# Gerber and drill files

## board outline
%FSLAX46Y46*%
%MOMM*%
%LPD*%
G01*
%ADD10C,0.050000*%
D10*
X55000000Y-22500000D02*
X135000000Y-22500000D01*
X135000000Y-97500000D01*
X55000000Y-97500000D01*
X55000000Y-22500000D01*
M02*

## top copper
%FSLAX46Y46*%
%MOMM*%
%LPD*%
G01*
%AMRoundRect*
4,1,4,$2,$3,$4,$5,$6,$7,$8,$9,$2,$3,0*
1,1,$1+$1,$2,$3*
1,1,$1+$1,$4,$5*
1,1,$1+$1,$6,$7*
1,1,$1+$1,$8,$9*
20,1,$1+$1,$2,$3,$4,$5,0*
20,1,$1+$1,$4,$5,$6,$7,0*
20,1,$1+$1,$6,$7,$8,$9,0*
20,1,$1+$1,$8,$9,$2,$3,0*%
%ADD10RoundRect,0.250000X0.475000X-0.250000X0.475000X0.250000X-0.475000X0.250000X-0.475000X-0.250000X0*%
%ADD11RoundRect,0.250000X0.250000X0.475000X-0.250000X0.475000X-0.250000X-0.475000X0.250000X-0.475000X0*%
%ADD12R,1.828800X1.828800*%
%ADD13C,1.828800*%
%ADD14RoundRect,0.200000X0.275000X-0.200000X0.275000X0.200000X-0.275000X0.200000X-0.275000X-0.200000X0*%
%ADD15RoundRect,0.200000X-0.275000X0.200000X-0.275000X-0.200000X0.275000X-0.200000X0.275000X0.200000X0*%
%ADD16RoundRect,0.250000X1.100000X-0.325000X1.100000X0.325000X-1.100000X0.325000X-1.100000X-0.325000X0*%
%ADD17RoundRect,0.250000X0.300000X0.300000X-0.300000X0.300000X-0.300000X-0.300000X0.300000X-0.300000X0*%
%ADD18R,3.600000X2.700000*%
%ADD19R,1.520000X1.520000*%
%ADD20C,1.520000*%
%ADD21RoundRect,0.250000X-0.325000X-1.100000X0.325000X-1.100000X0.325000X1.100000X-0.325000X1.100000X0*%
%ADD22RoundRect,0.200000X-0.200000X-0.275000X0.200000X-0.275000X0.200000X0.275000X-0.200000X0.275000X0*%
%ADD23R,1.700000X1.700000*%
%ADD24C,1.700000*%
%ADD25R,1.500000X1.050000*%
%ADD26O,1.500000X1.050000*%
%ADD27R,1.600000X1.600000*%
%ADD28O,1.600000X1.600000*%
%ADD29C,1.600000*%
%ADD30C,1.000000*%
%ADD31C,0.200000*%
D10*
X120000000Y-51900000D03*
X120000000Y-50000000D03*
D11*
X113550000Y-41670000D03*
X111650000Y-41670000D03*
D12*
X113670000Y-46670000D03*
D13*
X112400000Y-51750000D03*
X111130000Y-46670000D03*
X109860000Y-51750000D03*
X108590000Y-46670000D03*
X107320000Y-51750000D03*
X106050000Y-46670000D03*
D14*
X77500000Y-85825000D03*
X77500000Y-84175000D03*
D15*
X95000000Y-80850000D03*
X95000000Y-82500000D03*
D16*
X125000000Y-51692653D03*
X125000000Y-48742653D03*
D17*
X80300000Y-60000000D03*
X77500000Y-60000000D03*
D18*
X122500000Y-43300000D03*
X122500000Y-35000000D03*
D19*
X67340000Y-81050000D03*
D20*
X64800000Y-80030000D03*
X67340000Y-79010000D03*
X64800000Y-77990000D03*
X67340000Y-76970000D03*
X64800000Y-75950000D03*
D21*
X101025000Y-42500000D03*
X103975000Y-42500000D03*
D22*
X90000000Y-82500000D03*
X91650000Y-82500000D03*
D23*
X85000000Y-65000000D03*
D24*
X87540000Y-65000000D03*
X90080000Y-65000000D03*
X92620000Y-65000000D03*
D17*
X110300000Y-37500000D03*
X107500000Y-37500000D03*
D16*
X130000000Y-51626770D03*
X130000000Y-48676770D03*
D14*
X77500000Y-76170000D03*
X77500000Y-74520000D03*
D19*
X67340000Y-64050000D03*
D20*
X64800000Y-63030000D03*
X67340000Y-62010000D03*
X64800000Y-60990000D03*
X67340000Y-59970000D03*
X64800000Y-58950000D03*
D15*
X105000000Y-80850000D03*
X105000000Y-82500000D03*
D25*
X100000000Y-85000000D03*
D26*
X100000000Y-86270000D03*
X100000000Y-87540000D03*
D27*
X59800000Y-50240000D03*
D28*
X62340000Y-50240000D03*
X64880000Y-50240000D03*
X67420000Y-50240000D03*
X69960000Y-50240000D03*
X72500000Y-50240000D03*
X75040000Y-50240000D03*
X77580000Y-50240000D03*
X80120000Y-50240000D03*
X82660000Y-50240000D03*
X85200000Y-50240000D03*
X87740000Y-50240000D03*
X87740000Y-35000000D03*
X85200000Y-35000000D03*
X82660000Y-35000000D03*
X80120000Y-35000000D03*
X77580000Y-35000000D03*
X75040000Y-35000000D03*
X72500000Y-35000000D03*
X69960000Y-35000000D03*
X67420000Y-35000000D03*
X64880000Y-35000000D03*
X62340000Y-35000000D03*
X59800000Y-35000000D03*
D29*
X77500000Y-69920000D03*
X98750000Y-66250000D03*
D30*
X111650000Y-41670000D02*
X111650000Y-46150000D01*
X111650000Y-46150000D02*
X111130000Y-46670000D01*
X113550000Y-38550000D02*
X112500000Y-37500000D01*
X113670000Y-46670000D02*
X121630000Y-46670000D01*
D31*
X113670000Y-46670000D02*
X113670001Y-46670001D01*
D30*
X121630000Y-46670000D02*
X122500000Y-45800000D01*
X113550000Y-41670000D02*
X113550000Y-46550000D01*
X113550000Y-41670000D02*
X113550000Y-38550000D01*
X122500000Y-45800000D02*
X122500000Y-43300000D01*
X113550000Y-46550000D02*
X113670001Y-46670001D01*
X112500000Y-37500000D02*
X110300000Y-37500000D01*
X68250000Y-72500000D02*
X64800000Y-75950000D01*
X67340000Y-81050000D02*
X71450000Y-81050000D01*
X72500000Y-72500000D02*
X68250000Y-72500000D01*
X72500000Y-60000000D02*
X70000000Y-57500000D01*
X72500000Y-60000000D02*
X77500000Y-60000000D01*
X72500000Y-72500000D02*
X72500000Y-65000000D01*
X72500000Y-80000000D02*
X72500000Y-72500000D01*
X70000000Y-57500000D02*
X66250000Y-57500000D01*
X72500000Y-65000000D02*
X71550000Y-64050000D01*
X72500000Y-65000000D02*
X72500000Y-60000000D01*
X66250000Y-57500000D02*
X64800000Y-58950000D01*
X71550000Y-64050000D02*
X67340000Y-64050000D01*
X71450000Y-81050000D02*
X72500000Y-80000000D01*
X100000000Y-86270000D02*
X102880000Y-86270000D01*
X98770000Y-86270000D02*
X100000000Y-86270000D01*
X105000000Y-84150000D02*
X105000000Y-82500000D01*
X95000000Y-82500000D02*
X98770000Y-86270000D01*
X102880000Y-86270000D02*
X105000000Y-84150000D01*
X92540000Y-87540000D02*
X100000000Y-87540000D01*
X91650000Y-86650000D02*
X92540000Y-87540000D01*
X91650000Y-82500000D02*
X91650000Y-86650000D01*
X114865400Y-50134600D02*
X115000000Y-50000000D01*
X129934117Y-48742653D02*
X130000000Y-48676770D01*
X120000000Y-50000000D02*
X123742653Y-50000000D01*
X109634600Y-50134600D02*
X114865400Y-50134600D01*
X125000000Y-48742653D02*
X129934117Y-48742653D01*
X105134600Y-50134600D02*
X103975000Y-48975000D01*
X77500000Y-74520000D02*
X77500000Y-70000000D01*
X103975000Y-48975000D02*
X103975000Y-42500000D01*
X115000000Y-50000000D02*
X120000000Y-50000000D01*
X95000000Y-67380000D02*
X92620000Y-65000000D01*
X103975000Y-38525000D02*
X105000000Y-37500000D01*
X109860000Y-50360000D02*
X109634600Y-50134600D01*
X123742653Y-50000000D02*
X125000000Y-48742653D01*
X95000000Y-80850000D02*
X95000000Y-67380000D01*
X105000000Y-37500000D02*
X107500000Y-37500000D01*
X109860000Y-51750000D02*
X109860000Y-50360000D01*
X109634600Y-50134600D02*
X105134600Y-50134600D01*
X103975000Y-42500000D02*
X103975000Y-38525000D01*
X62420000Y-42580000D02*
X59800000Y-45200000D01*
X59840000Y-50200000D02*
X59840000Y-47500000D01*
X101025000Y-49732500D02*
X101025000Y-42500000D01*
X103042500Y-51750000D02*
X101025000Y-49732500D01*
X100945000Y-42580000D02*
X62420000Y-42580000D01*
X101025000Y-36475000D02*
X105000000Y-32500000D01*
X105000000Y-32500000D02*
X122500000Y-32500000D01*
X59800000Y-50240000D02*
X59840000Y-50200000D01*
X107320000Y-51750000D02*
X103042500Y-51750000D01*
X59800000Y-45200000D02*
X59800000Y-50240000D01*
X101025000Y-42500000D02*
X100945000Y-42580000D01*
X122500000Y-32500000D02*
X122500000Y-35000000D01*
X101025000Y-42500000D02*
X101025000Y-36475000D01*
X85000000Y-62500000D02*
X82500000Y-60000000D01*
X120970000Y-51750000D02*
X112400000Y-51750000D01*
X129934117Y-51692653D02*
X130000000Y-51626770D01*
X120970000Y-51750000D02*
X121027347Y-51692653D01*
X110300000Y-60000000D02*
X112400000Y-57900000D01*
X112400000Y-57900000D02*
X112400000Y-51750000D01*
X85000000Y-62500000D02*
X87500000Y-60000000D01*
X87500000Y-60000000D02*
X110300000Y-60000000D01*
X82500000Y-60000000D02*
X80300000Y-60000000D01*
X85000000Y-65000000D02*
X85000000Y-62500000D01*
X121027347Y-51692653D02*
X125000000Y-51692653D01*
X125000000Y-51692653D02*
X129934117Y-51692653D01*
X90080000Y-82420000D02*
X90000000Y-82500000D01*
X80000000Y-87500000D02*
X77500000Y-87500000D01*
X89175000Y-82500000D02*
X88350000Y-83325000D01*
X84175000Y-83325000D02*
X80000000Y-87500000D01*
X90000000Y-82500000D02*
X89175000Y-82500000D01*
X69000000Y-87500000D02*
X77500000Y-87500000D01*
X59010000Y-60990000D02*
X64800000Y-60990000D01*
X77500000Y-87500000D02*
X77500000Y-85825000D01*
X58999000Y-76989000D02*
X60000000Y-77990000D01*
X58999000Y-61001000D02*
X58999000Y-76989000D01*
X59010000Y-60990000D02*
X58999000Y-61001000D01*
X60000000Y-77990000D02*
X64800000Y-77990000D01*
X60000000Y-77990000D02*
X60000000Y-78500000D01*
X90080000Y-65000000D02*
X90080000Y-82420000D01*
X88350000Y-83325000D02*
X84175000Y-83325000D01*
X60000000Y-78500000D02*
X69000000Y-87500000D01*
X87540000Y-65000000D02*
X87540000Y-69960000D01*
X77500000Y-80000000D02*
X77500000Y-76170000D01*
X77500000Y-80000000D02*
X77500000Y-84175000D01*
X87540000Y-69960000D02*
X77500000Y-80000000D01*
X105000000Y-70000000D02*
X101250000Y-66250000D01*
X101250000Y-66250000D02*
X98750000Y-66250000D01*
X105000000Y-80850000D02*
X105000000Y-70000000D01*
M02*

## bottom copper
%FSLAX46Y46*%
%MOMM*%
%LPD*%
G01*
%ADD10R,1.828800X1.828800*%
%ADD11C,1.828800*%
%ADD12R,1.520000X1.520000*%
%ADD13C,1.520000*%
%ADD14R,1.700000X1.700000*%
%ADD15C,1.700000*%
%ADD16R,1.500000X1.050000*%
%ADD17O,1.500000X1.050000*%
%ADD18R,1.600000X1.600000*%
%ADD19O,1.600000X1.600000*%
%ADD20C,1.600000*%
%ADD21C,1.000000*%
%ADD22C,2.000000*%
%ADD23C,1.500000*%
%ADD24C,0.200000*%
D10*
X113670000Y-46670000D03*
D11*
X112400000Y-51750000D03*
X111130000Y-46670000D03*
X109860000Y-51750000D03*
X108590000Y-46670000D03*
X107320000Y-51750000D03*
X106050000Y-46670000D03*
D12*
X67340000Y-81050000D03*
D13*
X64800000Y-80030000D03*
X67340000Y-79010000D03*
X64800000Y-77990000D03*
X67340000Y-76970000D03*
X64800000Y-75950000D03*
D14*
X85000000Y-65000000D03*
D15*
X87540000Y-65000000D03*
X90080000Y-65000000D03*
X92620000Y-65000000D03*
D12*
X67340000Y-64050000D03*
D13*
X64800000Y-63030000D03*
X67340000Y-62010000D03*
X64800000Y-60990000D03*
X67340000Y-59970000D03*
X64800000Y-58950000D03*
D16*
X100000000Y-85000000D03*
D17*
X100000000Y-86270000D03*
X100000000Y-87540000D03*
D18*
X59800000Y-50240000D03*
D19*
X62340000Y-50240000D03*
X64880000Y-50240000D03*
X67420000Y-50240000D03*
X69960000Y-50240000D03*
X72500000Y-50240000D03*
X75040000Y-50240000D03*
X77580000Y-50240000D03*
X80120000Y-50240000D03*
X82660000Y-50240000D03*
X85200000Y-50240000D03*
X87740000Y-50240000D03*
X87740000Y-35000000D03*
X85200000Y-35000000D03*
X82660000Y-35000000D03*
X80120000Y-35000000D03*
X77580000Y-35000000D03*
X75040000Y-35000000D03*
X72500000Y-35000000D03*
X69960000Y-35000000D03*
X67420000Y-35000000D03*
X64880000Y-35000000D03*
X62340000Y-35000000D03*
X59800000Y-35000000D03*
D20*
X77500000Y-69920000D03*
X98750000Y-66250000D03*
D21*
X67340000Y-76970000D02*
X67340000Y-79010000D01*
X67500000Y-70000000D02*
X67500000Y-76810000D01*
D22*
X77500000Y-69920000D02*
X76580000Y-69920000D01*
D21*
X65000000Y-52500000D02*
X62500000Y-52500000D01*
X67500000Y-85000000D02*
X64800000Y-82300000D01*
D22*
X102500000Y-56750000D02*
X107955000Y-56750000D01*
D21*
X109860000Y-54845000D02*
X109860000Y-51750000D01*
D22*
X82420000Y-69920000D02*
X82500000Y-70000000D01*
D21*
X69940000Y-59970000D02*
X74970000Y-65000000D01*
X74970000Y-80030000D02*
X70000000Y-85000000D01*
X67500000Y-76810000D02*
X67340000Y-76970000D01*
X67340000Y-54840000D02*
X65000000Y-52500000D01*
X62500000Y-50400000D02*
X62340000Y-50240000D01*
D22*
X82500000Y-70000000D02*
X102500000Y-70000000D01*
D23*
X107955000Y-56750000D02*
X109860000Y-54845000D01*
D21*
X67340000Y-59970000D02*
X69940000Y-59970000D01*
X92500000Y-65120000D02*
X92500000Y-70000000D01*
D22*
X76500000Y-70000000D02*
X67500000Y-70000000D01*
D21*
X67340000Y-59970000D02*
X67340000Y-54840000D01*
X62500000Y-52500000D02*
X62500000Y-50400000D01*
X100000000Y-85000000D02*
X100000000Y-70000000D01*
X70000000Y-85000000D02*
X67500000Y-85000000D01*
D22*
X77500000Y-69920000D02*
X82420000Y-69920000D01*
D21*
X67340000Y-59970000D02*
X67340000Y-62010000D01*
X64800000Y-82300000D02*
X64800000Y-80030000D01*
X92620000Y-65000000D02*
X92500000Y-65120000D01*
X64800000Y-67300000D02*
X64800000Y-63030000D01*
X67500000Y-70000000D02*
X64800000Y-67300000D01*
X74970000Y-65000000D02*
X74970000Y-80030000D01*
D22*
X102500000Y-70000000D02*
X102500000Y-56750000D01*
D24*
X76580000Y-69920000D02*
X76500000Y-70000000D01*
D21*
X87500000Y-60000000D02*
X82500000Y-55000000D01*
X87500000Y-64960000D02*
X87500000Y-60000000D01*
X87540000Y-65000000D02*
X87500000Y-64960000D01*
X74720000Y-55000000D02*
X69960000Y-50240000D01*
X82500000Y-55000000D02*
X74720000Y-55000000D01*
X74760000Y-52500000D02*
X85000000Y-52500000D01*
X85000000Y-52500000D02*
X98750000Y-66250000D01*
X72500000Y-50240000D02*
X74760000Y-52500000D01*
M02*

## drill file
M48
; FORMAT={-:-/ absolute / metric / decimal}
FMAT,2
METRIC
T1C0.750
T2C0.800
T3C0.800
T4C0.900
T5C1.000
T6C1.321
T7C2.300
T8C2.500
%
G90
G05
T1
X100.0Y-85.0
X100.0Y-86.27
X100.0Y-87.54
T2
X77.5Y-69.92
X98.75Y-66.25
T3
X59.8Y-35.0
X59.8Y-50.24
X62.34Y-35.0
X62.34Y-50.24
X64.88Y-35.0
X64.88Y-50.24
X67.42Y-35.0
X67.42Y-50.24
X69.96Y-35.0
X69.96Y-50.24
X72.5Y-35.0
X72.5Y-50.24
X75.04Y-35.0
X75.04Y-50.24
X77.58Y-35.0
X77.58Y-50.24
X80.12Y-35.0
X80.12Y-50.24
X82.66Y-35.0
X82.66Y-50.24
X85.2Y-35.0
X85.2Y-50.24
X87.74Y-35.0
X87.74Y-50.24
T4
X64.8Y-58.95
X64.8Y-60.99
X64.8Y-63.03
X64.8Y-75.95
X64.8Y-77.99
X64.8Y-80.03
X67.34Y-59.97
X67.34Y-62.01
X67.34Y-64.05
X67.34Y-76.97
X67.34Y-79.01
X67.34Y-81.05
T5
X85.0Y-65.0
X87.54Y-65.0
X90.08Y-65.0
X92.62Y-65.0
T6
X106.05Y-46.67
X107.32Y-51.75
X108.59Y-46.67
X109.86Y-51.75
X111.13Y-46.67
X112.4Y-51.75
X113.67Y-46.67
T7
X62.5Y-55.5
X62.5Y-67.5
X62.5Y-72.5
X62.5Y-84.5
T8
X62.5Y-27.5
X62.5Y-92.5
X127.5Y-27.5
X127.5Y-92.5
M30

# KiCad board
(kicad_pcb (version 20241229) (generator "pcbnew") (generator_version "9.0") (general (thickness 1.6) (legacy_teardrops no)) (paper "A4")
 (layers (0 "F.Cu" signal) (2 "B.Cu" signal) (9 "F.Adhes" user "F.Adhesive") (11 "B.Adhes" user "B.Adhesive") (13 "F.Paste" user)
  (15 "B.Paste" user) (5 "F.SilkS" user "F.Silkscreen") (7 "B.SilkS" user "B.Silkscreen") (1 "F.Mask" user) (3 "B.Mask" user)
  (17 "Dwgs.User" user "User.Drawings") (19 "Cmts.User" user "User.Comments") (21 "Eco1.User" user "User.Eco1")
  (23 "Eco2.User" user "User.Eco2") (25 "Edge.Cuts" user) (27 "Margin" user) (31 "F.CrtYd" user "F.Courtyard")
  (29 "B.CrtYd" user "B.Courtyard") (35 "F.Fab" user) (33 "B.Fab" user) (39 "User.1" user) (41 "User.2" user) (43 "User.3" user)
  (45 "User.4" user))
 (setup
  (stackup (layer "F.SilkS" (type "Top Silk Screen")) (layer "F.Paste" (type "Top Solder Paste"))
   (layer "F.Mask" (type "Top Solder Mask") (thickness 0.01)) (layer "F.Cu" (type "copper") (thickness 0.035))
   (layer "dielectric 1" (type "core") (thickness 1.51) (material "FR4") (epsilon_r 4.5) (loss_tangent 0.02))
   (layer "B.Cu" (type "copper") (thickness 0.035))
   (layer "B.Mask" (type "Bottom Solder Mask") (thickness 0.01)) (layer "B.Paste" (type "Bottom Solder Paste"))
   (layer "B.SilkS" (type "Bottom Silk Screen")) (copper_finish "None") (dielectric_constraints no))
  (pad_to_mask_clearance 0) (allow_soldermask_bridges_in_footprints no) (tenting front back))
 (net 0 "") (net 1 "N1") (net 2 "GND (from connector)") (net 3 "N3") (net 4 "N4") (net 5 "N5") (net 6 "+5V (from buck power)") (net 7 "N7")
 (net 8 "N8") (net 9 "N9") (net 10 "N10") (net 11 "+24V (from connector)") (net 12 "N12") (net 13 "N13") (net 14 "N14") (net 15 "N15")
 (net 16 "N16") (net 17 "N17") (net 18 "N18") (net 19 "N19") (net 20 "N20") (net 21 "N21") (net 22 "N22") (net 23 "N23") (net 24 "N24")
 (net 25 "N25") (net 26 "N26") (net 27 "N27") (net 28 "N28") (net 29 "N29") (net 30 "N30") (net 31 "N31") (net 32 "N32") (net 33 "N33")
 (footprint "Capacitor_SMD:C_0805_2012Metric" (layer "F.Cu") (at 120 50.95 90)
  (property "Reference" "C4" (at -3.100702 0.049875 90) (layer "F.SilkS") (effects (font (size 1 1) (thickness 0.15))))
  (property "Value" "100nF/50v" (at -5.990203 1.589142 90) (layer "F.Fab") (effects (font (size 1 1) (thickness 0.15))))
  (pad "1" smd roundrect (at -0.95 0 90) (size 1 1.45) (layers "F.Cu" "F.Mask" "F.Paste") (roundrect_rratio 0.25) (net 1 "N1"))
  (pad "2" smd roundrect (at 0.95 0 90) (size 1 1.45) (layers "F.Cu" "F.Mask" "F.Paste") (roundrect_rratio 0.25)
   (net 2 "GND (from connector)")))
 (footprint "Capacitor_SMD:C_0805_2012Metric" (layer "F.Cu") (at 112.6 41.67 180)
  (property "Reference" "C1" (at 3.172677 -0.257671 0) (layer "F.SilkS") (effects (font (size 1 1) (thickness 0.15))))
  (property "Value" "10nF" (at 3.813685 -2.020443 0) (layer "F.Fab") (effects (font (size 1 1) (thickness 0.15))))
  (pad "1" smd roundrect (at -0.95 0 180) (size 1 1.45) (layers "F.Cu" "F.Mask" "F.Paste") (roundrect_rratio 0.25) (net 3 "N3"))
  (pad "2" smd roundrect (at 0.95 0 180) (size 1 1.45) (layers "F.Cu" "F.Mask" "F.Paste") (roundrect_rratio 0.25) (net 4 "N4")))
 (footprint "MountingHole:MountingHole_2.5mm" (layer "F.Cu") (at 62.5 27.5)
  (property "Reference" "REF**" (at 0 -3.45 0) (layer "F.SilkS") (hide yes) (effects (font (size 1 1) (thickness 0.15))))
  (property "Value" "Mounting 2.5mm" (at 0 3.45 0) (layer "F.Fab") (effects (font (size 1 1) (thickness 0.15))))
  (pad "" np_thru_hole circle (at 0 0) (size 2.5 2.5) (drill 2.5) (layers "*.Cu" "*.Mask")))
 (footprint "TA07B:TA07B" (layer "F.Cu") (at 106.05 57.8714 180)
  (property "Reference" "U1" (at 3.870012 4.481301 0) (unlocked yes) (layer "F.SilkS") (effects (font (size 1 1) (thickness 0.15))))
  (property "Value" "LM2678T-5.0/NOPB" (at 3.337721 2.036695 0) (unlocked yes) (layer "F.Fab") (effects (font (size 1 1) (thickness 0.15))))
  (pad "1" thru_hole rect (at -7.62 11.2014 180) (size 1.8288 1.8288) (drill 1.3208) (layers "*.Cu" "*.Mask") (remove_unused_layers no)
   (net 3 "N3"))
  (pad "2" thru_hole circle (at -6.35 6.1214 180) (size 1.8288 1.8288) (drill 1.3208) (layers "*.Cu" "*.Mask") (remove_unused_layers no)
   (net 1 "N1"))
  (pad "3" thru_hole circle (at -5.08 11.2014 180) (size 1.8288 1.8288) (drill 1.3208) (layers "*.Cu" "*.Mask") (remove_unused_layers no)
   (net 4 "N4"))
  (pad "4" thru_hole circle (at -3.81 6.1214 180) (size 1.8288 1.8288) (drill 1.3208) (layers "*.Cu" "*.Mask") (remove_unused_layers no)
   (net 2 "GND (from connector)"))
  (pad "5" thru_hole circle (at -2.54 11.2014 180) (size 1.8288 1.8288) (drill 1.3208) (layers "*.Cu" "*.Mask") (remove_unused_layers no)
   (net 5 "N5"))
  (pad "6" thru_hole circle (at -1.27 6.1214 180) (size 1.8288 1.8288) (drill 1.3208) (layers "*.Cu" "*.Mask") (remove_unused_layers no)
   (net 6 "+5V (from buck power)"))
  (pad "7" thru_hole circle (at 0 11.2014 180) (size 1.8288 1.8288) (drill 1.3208) (layers "*.Cu" "*.Mask") (remove_unused_layers no)
   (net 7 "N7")))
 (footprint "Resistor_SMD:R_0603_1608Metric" (layer "F.Cu") (at 77.5 85 90)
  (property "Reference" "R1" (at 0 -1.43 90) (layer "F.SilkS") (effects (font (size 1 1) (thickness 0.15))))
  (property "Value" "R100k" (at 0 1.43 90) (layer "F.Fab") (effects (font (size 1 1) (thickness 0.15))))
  (pad "1" smd roundrect (at -0.825 0 90) (size 0.8 0.95) (layers "F.Cu" "F.Mask" "F.Paste") (roundrect_rratio 0.25) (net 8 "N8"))
  (pad "2" smd roundrect (at 0.825 0 90) (size 0.8 0.95) (layers "F.Cu" "F.Mask" "F.Paste") (roundrect_rratio 0.25) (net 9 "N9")))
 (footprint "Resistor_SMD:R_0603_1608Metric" (layer "F.Cu") (at 95 81.675 -90)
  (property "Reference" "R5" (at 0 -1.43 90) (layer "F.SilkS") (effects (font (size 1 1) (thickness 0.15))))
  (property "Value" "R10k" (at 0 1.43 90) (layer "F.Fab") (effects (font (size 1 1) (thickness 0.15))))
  (pad "1" smd roundrect (at -0.825 0 270) (size 0.8 0.95) (layers "F.Cu" "F.Mask" "F.Paste") (roundrect_rratio 0.25)
   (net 2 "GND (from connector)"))
  (pad "2" smd roundrect (at 0.825 0 270) (size 0.8 0.95) (layers "F.Cu" "F.Mask" "F.Paste") (roundrect_rratio 0.25) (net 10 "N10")))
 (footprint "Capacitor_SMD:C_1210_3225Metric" (layer "F.Cu") (at 125 50.217653 90)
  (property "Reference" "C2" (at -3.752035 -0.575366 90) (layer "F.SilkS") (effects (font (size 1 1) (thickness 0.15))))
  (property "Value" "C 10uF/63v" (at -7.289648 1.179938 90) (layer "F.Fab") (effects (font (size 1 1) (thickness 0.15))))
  (pad "1" smd roundrect (at -1.475 0 90) (size 1.15 2.7) (layers "F.Cu" "F.Mask" "F.Paste") (roundrect_rratio 0.217391) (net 1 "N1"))
  (pad "2" smd roundrect (at 1.475 0 90) (size 1.15 2.7) (layers "F.Cu" "F.Mask" "F.Paste") (roundrect_rratio 0.217391)
   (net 2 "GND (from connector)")))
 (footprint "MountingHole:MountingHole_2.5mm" (layer "F.Cu") (at 127.5 27.5)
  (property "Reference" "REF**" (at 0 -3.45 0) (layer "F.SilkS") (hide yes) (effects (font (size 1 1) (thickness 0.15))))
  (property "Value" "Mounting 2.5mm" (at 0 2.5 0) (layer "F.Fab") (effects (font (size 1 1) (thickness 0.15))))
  (pad "" np_thru_hole circle (at 0 0) (size 2.5 2.5) (drill 2.5) (layers "*.Cu" "*.Mask")))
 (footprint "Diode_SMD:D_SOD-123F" (layer "F.Cu") (at 78.9 60 180)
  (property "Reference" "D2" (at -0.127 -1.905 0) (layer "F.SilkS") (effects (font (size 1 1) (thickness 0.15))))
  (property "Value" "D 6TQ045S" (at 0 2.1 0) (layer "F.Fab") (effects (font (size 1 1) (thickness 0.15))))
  (pad "1" smd roundrect (at -1.4 0 180) (size 1.1 1.1) (layers "F.Cu" "F.Mask" "F.Paste") (roundrect_rratio 0.2272727273) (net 1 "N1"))
  (pad "2" smd roundrect (at 1.4 0 180) (size 1.1 1.1) (layers "F.Cu" "F.Mask" "F.Paste") (roundrect_rratio 0.2272727273)
   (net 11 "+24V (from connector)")))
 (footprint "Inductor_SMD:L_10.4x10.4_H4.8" (layer "F.Cu") (at 122.5 39.15 90)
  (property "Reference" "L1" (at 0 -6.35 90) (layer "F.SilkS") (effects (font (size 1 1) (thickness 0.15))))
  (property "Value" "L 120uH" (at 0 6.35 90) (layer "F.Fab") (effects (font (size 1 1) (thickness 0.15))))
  (pad "1" smd rect (at -4.15 0 90) (size 2.7 3.6) (layers "F.Cu" "F.Mask" "F.Paste") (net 3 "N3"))
  (pad "2" smd rect (at 4.15 0 90) (size 2.7 3.6) (layers "F.Cu" "F.Mask" "F.Paste") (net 6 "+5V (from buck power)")))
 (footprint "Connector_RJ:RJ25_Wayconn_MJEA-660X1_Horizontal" (layer "F.Cu") (at 67.34 81.05 -90)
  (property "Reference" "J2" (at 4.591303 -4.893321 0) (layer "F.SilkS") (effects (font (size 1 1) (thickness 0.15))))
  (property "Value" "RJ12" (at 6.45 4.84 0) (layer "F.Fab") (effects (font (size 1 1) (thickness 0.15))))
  (pad "" np_thru_hole circle (at -8.55 4.84 270) (size 2.3 2.3) (drill 2.3) (layers "*.Cu" "*.Mask"))
  (pad "" np_thru_hole circle (at 3.45 4.84 270) (size 2.3 2.3) (drill 2.3) (layers "*.Cu" "*.Mask"))
  (pad "1" thru_hole rect (at 0 0 270) (size 1.52 1.52) (drill 0.9) (layers "*.Cu" "*.Mask") (remove_unused_layers no)
   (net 11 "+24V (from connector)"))
  (pad "2" thru_hole circle (at -1.02 2.54 270) (size 1.52 1.52) (drill 0.9) (layers "*.Cu" "*.Mask") (remove_unused_layers no)
   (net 2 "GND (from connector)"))
  (pad "3" thru_hole circle (at -2.04 0 270) (size 1.52 1.52) (drill 0.9) (layers "*.Cu" "*.Mask") (remove_unused_layers no)
   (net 2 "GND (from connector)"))
  (pad "4" thru_hole circle (at -3.06 2.54 270) (size 1.52 1.52) (drill 0.9) (layers "*.Cu" "*.Mask") (remove_unused_layers no) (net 8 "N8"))
  (pad "5" thru_hole circle (at -4.08 0 270) (size 1.52 1.52) (drill 0.9) (layers "*.Cu" "*.Mask") (remove_unused_layers no)
   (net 2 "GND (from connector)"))
  (pad "6" thru_hole circle (at -5.1 2.54 270) (size 1.52 1.52) (drill 0.9) (layers "*.Cu" "*.Mask") (remove_unused_layers no)
   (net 11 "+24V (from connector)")))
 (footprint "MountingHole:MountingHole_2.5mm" (layer "F.Cu") (at 127.5 92.5)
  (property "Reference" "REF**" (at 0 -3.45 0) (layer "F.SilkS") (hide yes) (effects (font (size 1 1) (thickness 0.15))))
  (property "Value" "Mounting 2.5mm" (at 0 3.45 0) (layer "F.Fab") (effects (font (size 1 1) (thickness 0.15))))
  (pad "" np_thru_hole circle (at 0 0) (size 2.5 2.5) (drill 2.5) (layers "*.Cu" "*.Mask")))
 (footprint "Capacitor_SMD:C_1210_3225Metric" (layer "F.Cu") (at 102.5 42.5)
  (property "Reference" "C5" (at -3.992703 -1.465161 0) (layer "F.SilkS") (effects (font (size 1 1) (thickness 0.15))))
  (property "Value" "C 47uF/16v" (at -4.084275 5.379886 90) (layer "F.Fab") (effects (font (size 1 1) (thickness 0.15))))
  (pad "1" smd roundrect (at -1.475 0) (size 1.15 2.7) (layers "F.Cu" "F.Mask" "F.Paste") (roundrect_rratio 0.217391)
   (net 6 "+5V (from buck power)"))
  (pad "2" smd roundrect (at 1.475 0) (size 1.15 2.7) (layers "F.Cu" "F.Mask" "F.Paste") (roundrect_rratio 0.217391)
   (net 2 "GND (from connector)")))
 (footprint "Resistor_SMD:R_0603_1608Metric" (layer "F.Cu") (at 90.825 82.5)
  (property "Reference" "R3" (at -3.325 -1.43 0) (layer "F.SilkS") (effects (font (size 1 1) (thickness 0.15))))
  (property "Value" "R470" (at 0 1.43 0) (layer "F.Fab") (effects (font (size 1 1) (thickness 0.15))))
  (pad "1" smd roundrect (at -0.825 0) (size 0.8 0.95) (layers "F.Cu" "F.Mask" "F.Paste") (roundrect_rratio 0.25) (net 8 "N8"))
  (pad "2" smd roundrect (at 0.825 0) (size 0.8 0.95) (layers "F.Cu" "F.Mask" "F.Paste") (roundrect_rratio 0.25) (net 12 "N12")))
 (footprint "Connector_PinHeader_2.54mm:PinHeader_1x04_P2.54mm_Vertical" (layer "F.Cu") (at 85 65 90)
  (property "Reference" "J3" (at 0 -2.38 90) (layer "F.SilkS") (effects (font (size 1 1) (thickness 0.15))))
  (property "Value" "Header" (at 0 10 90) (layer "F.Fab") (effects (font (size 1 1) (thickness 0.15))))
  (pad "1" thru_hole rect (at 0 0 90) (size 1.7 1.7) (drill 1) (layers "*.Cu" "*.Mask") (remove_unused_layers no) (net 1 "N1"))
  (pad "2" thru_hole circle (at 0 2.54 90) (size 1.7 1.7) (drill 1) (layers "*.Cu" "*.Mask") (remove_unused_layers no) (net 9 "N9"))
  (pad "3" thru_hole circle (at 0 5.08 90) (size 1.7 1.7) (drill 1) (layers "*.Cu" "*.Mask") (remove_unused_layers no) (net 8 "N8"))
  (pad "4" thru_hole circle (at 0 7.62 90) (size 1.7 1.7) (drill 1) (layers "*.Cu" "*.Mask") (remove_unused_layers no)
   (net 2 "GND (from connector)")))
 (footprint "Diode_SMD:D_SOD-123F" (layer "F.Cu") (at 108.9 37.5 180)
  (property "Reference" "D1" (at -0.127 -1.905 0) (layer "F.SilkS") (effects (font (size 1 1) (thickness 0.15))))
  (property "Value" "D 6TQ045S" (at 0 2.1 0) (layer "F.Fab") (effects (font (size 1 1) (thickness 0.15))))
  (pad "1" smd roundrect (at -1.4 0 180) (size 1.1 1.1) (layers "F.Cu" "F.Mask" "F.Paste") (roundrect_rratio 0.2272727273) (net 3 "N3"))
  (pad "2" smd roundrect (at 1.4 0 180) (size 1.1 1.1) (layers "F.Cu" "F.Mask" "F.Paste") (roundrect_rratio 0.2272727273)
   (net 2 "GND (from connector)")))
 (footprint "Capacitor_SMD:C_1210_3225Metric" (layer "F.Cu") (at 130 50.15177 90)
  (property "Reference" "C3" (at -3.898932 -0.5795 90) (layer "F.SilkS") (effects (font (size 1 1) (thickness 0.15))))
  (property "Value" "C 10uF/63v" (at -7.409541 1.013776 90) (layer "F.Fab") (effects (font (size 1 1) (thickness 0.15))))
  (pad "1" smd roundrect (at -1.475 0 90) (size 1.15 2.7) (layers "F.Cu" "F.Mask" "F.Paste") (roundrect_rratio 0.217391) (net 1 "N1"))
  (pad "2" smd roundrect (at 1.475 0 90) (size 1.15 2.7) (layers "F.Cu" "F.Mask" "F.Paste") (roundrect_rratio 0.217391)
   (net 2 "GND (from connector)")))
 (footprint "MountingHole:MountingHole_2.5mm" (layer "F.Cu") (at 62.5 92.5)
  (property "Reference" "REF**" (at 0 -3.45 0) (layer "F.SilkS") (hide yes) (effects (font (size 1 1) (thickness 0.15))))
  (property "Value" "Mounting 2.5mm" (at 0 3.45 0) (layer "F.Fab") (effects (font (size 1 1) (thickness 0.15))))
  (pad "" np_thru_hole circle (at 0 0) (size 2.5 2.5) (drill 2.5) (layers "*.Cu" "*.Mask")))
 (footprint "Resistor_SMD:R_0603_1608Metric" (layer "F.Cu") (at 77.5 75.345 90)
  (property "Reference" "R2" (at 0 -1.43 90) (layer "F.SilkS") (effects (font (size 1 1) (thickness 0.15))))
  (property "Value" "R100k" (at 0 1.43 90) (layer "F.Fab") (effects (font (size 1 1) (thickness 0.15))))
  (pad "1" smd roundrect (at -0.825 0 90) (size 0.8 0.95) (layers "F.Cu" "F.Mask" "F.Paste") (roundrect_rratio 0.25) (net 9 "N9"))
  (pad "2" smd roundrect (at 0.825 0 90) (size 0.8 0.95) (layers "F.Cu" "F.Mask" "F.Paste") (roundrect_rratio 0.25)
   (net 2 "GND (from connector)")))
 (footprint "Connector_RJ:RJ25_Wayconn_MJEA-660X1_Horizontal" (layer "F.Cu") (at 67.34 64.05 -90)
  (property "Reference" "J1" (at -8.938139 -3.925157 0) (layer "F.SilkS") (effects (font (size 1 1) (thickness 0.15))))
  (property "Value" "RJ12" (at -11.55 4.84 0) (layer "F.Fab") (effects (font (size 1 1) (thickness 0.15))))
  (pad "" np_thru_hole circle (at -8.55 4.84 270) (size 2.3 2.3) (drill 2.3) (layers "*.Cu" "*.Mask"))
  (pad "" np_thru_hole circle (at 3.45 4.84 270) (size 2.3 2.3) (drill 2.3) (layers "*.Cu" "*.Mask"))
  (pad "1" thru_hole rect (at 0 0 270) (size 1.52 1.52) (drill 0.9) (layers "*.Cu" "*.Mask") (remove_unused_layers no)
   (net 11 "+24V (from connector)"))
  (pad "2" thru_hole circle (at -1.02 2.54 270) (size 1.52 1.52) (drill 0.9) (layers "*.Cu" "*.Mask") (remove_unused_layers no)
   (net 2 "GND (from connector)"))
  (pad "3" thru_hole circle (at -2.04 0 270) (size 1.52 1.52) (drill 0.9) (layers "*.Cu" "*.Mask") (remove_unused_layers no)
   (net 2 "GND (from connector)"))
  (pad "4" thru_hole circle (at -3.06 2.54 270) (size 1.52 1.52) (drill 0.9) (layers "*.Cu" "*.Mask") (remove_unused_layers no) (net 8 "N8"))
  (pad "5" thru_hole circle (at -4.08 0 270) (size 1.52 1.52) (drill 0.9) (layers "*.Cu" "*.Mask") (remove_unused_layers no)
   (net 2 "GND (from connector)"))
  (pad "6" thru_hole circle (at -5.1 2.54 270) (size 1.52 1.52) (drill 0.9) (layers "*.Cu" "*.Mask") (remove_unused_layers no)
   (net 11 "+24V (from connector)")))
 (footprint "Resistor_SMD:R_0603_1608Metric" (layer "F.Cu") (at 105 81.675 -90)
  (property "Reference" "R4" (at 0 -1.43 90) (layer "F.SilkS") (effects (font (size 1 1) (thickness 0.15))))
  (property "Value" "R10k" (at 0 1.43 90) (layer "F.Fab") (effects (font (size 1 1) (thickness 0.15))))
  (pad "1" smd roundrect (at -0.825 0 270) (size 0.8 0.95) (layers "F.Cu" "F.Mask" "F.Paste") (roundrect_rratio 0.25) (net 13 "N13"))
  (pad "2" smd roundrect (at 0.825 0 270) (size 0.8 0.95) (layers "F.Cu" "F.Mask" "F.Paste") (roundrect_rratio 0.25) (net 10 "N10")))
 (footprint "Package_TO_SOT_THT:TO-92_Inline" (layer "F.Cu") (at 100 85 -90)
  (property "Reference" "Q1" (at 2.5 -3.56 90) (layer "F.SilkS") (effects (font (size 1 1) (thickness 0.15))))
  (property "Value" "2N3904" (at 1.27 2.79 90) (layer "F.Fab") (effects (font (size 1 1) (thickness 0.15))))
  (pad "1" thru_hole rect (at 0 0 270) (size 1.05 1.5) (drill 0.75) (layers "*.Cu" "*.Mask") (remove_unused_layers no)
   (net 2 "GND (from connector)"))
  (pad "2" thru_hole oval (at 1.27 0 270) (size 1.05 1.5) (drill 0.75) (layers "*.Cu" "*.Mask") (remove_unused_layers no) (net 10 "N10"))
  (pad "3" thru_hole oval (at 2.54 0 270) (size 1.05 1.5) (drill 0.75) (layers "*.Cu" "*.Mask") (remove_unused_layers no) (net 12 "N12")))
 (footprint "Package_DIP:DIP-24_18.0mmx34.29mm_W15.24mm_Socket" (layer "F.Cu") (at 59.8 50.24 90)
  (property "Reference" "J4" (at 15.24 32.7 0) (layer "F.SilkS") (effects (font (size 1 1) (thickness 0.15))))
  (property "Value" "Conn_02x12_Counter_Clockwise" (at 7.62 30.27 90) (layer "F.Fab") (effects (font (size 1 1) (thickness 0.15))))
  (pad "1" thru_hole rect (at 0 0 90) (size 1.6 1.6) (drill 0.8) (layers "*.Cu" "*.Mask") (remove_unused_layers no)
   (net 6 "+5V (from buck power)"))
  (pad "2" thru_hole oval (at 0 2.54 90) (size 1.6 1.6) (drill 0.8) (layers "*.Cu" "*.Mask") (remove_unused_layers no)
   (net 2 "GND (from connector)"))
  (pad "3" thru_hole oval (at 0 5.08 90) (size 1.6 1.6) (drill 0.8) (layers "*.Cu" "*.Mask") (remove_unused_layers no) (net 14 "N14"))
  (pad "4" thru_hole oval (at 0 7.62 90) (size 1.6 1.6) (drill 0.8) (layers "*.Cu" "*.Mask") (remove_unused_layers no) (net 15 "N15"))
  (pad "5" thru_hole oval (at 0 10.16 90) (size 1.6 1.6) (drill 0.8) (layers "*.Cu" "*.Mask") (remove_unused_layers no) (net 9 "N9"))
  (pad "6" thru_hole oval (at 0 12.7 90) (size 1.6 1.6) (drill 0.8) (layers "*.Cu" "*.Mask") (remove_unused_layers no) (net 13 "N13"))
  (pad "7" thru_hole oval (at 0 15.24 90) (size 1.6 1.6) (drill 0.8) (layers "*.Cu" "*.Mask") (remove_unused_layers no) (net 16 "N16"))
  (pad "8" thru_hole oval (at 0 17.78 90) (size 1.6 1.6) (drill 0.8) (layers "*.Cu" "*.Mask") (remove_unused_layers no) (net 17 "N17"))
  (pad "9" thru_hole oval (at 0 20.32 90) (size 1.6 1.6) (drill 0.8) (layers "*.Cu" "*.Mask") (remove_unused_layers no) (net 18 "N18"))
  (pad "10" thru_hole oval (at 0 22.86 90) (size 1.6 1.6) (drill 0.8) (layers "*.Cu" "*.Mask") (remove_unused_layers no) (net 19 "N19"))
  (pad "11" thru_hole oval (at 0 25.4 90) (size 1.6 1.6) (drill 0.8) (layers "*.Cu" "*.Mask") (remove_unused_layers no) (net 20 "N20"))
  (pad "12" thru_hole oval (at 0 27.94 90) (size 1.6 1.6) (drill 0.8) (layers "*.Cu" "*.Mask") (remove_unused_layers no) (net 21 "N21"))
  (pad "13" thru_hole oval (at 15.24 27.94 90) (size 1.6 1.6) (drill 0.8) (layers "*.Cu" "*.Mask") (remove_unused_layers no) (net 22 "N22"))
  (pad "14" thru_hole oval (at 15.24 25.4 90) (size 1.6 1.6) (drill 0.8) (layers "*.Cu" "*.Mask") (remove_unused_layers no) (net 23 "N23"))
  (pad "15" thru_hole oval (at 15.24 22.86 90) (size 1.6 1.6) (drill 0.8) (layers "*.Cu" "*.Mask") (remove_unused_layers no) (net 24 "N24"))
  (pad "16" thru_hole oval (at 15.24 20.32 90) (size 1.6 1.6) (drill 0.8) (layers "*.Cu" "*.Mask") (remove_unused_layers no) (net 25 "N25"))
  (pad "17" thru_hole oval (at 15.24 17.78 90) (size 1.6 1.6) (drill 0.8) (layers "*.Cu" "*.Mask") (remove_unused_layers no) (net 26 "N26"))
  (pad "18" thru_hole oval (at 15.24 15.24 90) (size 1.6 1.6) (drill 0.8) (layers "*.Cu" "*.Mask") (remove_unused_layers no) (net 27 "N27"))
  (pad "19" thru_hole oval (at 15.24 12.7 90) (size 1.6 1.6) (drill 0.8) (layers "*.Cu" "*.Mask") (remove_unused_layers no) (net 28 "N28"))
  (pad "20" thru_hole oval (at 15.24 10.16 90) (size 1.6 1.6) (drill 0.8) (layers "*.Cu" "*.Mask") (remove_unused_layers no) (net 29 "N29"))
  (pad "21" thru_hole oval (at 15.24 7.62 90) (size 1.6 1.6) (drill 0.8) (layers "*.Cu" "*.Mask") (remove_unused_layers no) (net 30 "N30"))
  (pad "22" thru_hole oval (at 15.24 5.08 90) (size 1.6 1.6) (drill 0.8) (layers "*.Cu" "*.Mask") (remove_unused_layers no) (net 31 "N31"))
  (pad "23" thru_hole oval (at 15.24 2.54 90) (size 1.6 1.6) (drill 0.8) (layers "*.Cu" "*.Mask") (remove_unused_layers no) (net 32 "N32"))
  (pad "24" thru_hole oval (at 15.24 0 90) (size 1.6 1.6) (drill 0.8) (layers "*.Cu" "*.Mask") (remove_unused_layers no) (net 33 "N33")))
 (gr_rect (start 55 22.5) (end 135 97.5) (stroke (width 0.05) (type default)) (fill no) (layer "Edge.Cuts"))
 (segment (start 111.65 41.67) (end 111.65 46.15) (width 1) (layer "F.Cu") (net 4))
 (segment (start 111.65 46.15) (end 111.13 46.67) (width 1) (layer "F.Cu") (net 4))
 (segment (start 113.55 38.55) (end 112.5 37.5) (width 1) (layer "F.Cu") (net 3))
 (segment (start 113.67 46.67) (end 121.63 46.67) (width 1) (layer "F.Cu") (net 3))
 (segment (start 113.67 46.67) (end 113.670001 46.670001) (width 0.2) (layer "F.Cu") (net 3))
 (segment (start 121.63 46.67) (end 122.5 45.8) (width 1) (layer "F.Cu") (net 3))
 (segment (start 113.55 41.67) (end 113.55 46.55) (width 1) (layer "F.Cu") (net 3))
 (segment (start 113.55 41.67) (end 113.55 38.55) (width 1) (layer "F.Cu") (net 3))
 (segment (start 122.5 45.8) (end 122.5 43.3) (width 1) (layer "F.Cu") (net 3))
 (segment (start 113.55 46.55) (end 113.670001 46.670001) (width 1) (layer "F.Cu") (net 3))
 (segment (start 112.5 37.5) (end 110.3 37.5) (width 1) (layer "F.Cu") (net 3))
 (segment (start 68.25 72.5) (end 64.8 75.95) (width 1) (layer "F.Cu") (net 11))
 (segment (start 67.34 81.05) (end 71.45 81.05) (width 1) (layer "F.Cu") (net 11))
 (segment (start 72.5 72.5) (end 68.25 72.5) (width 1) (layer "F.Cu") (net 11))
 (segment (start 72.5 60) (end 70 57.5) (width 1) (layer "F.Cu") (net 11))
 (segment (start 72.5 60) (end 77.5 60) (width 1) (layer "F.Cu") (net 11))
 (segment (start 72.5 72.5) (end 72.5 65) (width 1) (layer "F.Cu") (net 11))
 (segment (start 72.5 80) (end 72.5 72.5) (width 1) (layer "F.Cu") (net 11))
 (segment (start 70 57.5) (end 66.25 57.5) (width 1) (layer "F.Cu") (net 11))
 (segment (start 72.5 65) (end 71.55 64.05) (width 1) (layer "F.Cu") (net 11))
 (segment (start 72.5 65) (end 72.5 60) (width 1) (layer "F.Cu") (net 11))
 (segment (start 66.25 57.5) (end 64.8 58.95) (width 1) (layer "F.Cu") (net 11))
 (segment (start 71.55 64.05) (end 67.34 64.05) (width 1) (layer "F.Cu") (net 11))
 (segment (start 71.45 81.05) (end 72.5 80) (width 1) (layer "F.Cu") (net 11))
 (segment (start 100 86.27) (end 102.88 86.27) (width 1) (layer "F.Cu") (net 10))
 (segment (start 98.77 86.27) (end 100 86.27) (width 1) (layer "F.Cu") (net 10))
 (segment (start 105 84.15) (end 105 82.5) (width 1) (layer "F.Cu") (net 10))
 (segment (start 95 82.5) (end 98.77 86.27) (width 1) (layer "F.Cu") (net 10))
 (segment (start 102.88 86.27) (end 105 84.15) (width 1) (layer "F.Cu") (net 10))
 (segment (start 92.54 87.54) (end 100 87.54) (width 1) (layer "F.Cu") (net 12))
 (segment (start 91.65 86.65) (end 92.54 87.54) (width 1) (layer "F.Cu") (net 12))
 (segment (start 91.65 82.5) (end 91.65 86.65) (width 1) (layer "F.Cu") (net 12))
 (segment (start 114.8654 50.1346) (end 115 50) (width 1) (layer "F.Cu") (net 2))
 (segment (start 129.934117 48.742653) (end 130 48.67677) (width 1) (layer "F.Cu") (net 2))
 (segment (start 120 50) (end 123.742653 50) (width 1) (layer "F.Cu") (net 2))
 (segment (start 109.6346 50.1346) (end 114.8654 50.1346) (width 1) (layer "F.Cu") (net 2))
 (segment (start 125 48.742653) (end 129.934117 48.742653) (width 1) (layer "F.Cu") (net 2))
 (segment (start 105.1346 50.1346) (end 103.975 48.975) (width 1) (layer "F.Cu") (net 2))
 (segment (start 77.5 74.52) (end 77.5 70) (width 1) (layer "F.Cu") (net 2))
 (segment (start 103.975 48.975) (end 103.975 42.5) (width 1) (layer "F.Cu") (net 2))
 (segment (start 115 50) (end 120 50) (width 1) (layer "F.Cu") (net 2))
 (segment (start 95 67.38) (end 92.62 65) (width 1) (layer "F.Cu") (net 2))
 (segment (start 103.975 38.525) (end 105 37.5) (width 1) (layer "F.Cu") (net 2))
 (segment (start 109.86 50.36) (end 109.6346 50.1346) (width 1) (layer "F.Cu") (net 2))
 (segment (start 123.742653 50) (end 125 48.742653) (width 1) (layer "F.Cu") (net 2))
 (segment (start 95 80.85) (end 95 67.38) (width 1) (layer "F.Cu") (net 2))
 (segment (start 105 37.5) (end 107.5 37.5) (width 1) (layer "F.Cu") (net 2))
 (segment (start 109.86 51.75) (end 109.86 50.36) (width 1) (layer "F.Cu") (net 2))
 (segment (start 109.6346 50.1346) (end 105.1346 50.1346) (width 1) (layer "F.Cu") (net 2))
 (segment (start 103.975 42.5) (end 103.975 38.525) (width 1) (layer "F.Cu") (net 2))
 (via (at 77.5 69.92) (size 1.6) (drill 0.8) (layers "F.Cu" "B.Cu") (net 2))
 (segment (start 67.34 76.97) (end 67.34 79.01) (width 1) (layer "B.Cu") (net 2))
 (segment (start 67.5 70) (end 67.5 76.81) (width 1) (layer "B.Cu") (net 2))
 (segment (start 77.5 69.92) (end 76.58 69.92) (width 2) (layer "B.Cu") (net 2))
 (segment (start 65 52.5) (end 62.5 52.5) (width 1) (layer "B.Cu") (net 2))
 (segment (start 67.5 85) (end 64.8 82.3) (width 1) (layer "B.Cu") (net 2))
 (segment (start 102.5 56.75) (end 107.955 56.75) (width 2) (layer "B.Cu") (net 2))
 (segment (start 109.86 54.845) (end 109.86 51.75) (width 1) (layer "B.Cu") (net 2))
 (segment (start 82.42 69.92) (end 82.5 70) (width 2) (layer "B.Cu") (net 2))
 (segment (start 69.94 59.97) (end 74.97 65) (width 1) (layer "B.Cu") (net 2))
 (segment (start 74.97 80.03) (end 70 85) (width 1) (layer "B.Cu") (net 2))
 (segment (start 67.5 76.81) (end 67.34 76.97) (width 1) (layer "B.Cu") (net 2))
 (segment (start 67.34 54.84) (end 65 52.5) (width 1) (layer "B.Cu") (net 2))
 (segment (start 62.5 50.4) (end 62.34 50.24) (width 1) (layer "B.Cu") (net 2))
 (segment (start 82.5 70) (end 102.5 70) (width 2) (layer "B.Cu") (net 2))
 (segment (start 107.955 56.75) (end 109.86 54.845) (width 1.5) (layer "B.Cu") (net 2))
 (segment (start 67.34 59.97) (end 69.94 59.97) (width 1) (layer "B.Cu") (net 2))
 (segment (start 92.5 65.12) (end 92.5 70) (width 1) (layer "B.Cu") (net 2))
 (segment (start 76.5 70) (end 67.5 70) (width 2) (layer "B.Cu") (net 2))
 (segment (start 67.34 59.97) (end 67.34 54.84) (width 1) (layer "B.Cu") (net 2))
 (segment (start 62.5 52.5) (end 62.5 50.4) (width 1) (layer "B.Cu") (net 2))
 (segment (start 100 85) (end 100 70) (width 1) (layer "B.Cu") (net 2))
 (segment (start 70 85) (end 67.5 85) (width 1) (layer "B.Cu") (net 2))
 (segment (start 77.5 69.92) (end 82.42 69.92) (width 2) (layer "B.Cu") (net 2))
 (segment (start 67.34 59.97) (end 67.34 62.01) (width 1) (layer "B.Cu") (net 2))
 (segment (start 64.8 82.3) (end 64.8 80.03) (width 1) (layer "B.Cu") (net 2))
 (segment (start 92.62 65) (end 92.5 65.12) (width 1) (layer "B.Cu") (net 2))
 (segment (start 64.8 67.3) (end 64.8 63.03) (width 1) (layer "B.Cu") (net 2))
 (segment (start 67.5 70) (end 64.8 67.3) (width 1) (layer "B.Cu") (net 2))
 (segment (start 74.97 65) (end 74.97 80.03) (width 1) (layer "B.Cu") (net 2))
 (segment (start 102.5 70) (end 102.5 56.75) (width 2) (layer "B.Cu") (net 2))
 (segment (start 76.58 69.92) (end 76.5 70) (width 0.2) (layer "B.Cu") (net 2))
 (segment (start 62.42 42.58) (end 59.8 45.2) (width 1) (layer "F.Cu") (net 6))
 (segment (start 59.84 50.2) (end 59.84 47.5) (width 1) (layer "F.Cu") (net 6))
 (segment (start 101.025 49.7325) (end 101.025 42.5) (width 1) (layer "F.Cu") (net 6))
 (segment (start 103.0425 51.75) (end 101.025 49.7325) (width 1) (layer "F.Cu") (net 6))
 (segment (start 100.945 42.58) (end 62.42 42.58) (width 1) (layer "F.Cu") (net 6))
 (segment (start 101.025 36.475) (end 105 32.5) (width 1) (layer "F.Cu") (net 6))
 (segment (start 105 32.5) (end 122.5 32.5) (width 1) (layer "F.Cu") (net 6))
 (segment (start 59.8 50.24) (end 59.84 50.2) (width 1) (layer "F.Cu") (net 6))
 (segment (start 107.32 51.75) (end 103.0425 51.75) (width 1) (layer "F.Cu") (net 6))
 (segment (start 59.8 45.2) (end 59.8 50.24) (width 1) (layer "F.Cu") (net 6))
 (segment (start 101.025 42.5) (end 100.945 42.58) (width 1) (layer "F.Cu") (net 6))
 (segment (start 122.5 32.5) (end 122.5 35) (width 1) (layer "F.Cu") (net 6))
 (segment (start 101.025 42.5) (end 101.025 36.475) (width 1) (layer "F.Cu") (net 6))
 (segment (start 85 62.5) (end 82.5 60) (width 1) (layer "F.Cu") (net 1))
 (segment (start 120.97 51.75) (end 112.4 51.75) (width 1) (layer "F.Cu") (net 1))
 (segment (start 129.934117 51.692653) (end 130 51.62677) (width 1) (layer "F.Cu") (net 1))
 (segment (start 120.97 51.75) (end 121.027347 51.692653) (width 1) (layer "F.Cu") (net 1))
 (segment (start 110.3 60) (end 112.4 57.9) (width 1) (layer "F.Cu") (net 1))
 (segment (start 112.4 57.9) (end 112.4 51.75) (width 1) (layer "F.Cu") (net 1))
 (segment (start 85 62.5) (end 87.5 60) (width 1) (layer "F.Cu") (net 1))
 (segment (start 87.5 60) (end 110.3 60) (width 1) (layer "F.Cu") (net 1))
 (segment (start 82.5 60) (end 80.3 60) (width 1) (layer "F.Cu") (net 1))
 (segment (start 85 65) (end 85 62.5) (width 1) (layer "F.Cu") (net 1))
 (segment (start 121.027347 51.692653) (end 125 51.692653) (width 1) (layer "F.Cu") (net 1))
 (segment (start 125 51.692653) (end 129.934117 51.692653) (width 1) (layer "F.Cu") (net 1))
 (segment (start 90.08 82.42) (end 90 82.5) (width 1) (layer "F.Cu") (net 8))
 (segment (start 80 87.5) (end 77.5 87.5) (width 1) (layer "F.Cu") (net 8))
 (segment (start 89.175 82.5) (end 88.35 83.325) (width 1) (layer "F.Cu") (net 8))
 (segment (start 84.175 83.325) (end 80 87.5) (width 1) (layer "F.Cu") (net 8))
 (segment (start 90 82.5) (end 89.175 82.5) (width 1) (layer "F.Cu") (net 8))
 (segment (start 69 87.5) (end 77.5 87.5) (width 1) (layer "F.Cu") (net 8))
 (segment (start 59.01 60.99) (end 64.8 60.99) (width 1) (layer "F.Cu") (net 8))
 (segment (start 77.5 87.5) (end 77.5 85.825) (width 1) (layer "F.Cu") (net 8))
 (segment (start 58.999 76.989) (end 60 77.99) (width 1) (layer "F.Cu") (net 8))
 (segment (start 58.999 61.001) (end 58.999 76.989) (width 1) (layer "F.Cu") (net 8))
 (segment (start 59.01 60.99) (end 58.999 61.001) (width 1) (layer "F.Cu") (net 8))
 (segment (start 60 77.99) (end 64.8 77.99) (width 1) (layer "F.Cu") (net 8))
 (segment (start 60 77.99) (end 60 78.5) (width 1) (layer "F.Cu") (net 8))
 (segment (start 90.08 65) (end 90.08 82.42) (width 1) (layer "F.Cu") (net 8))
 (segment (start 88.35 83.325) (end 84.175 83.325) (width 1) (layer "F.Cu") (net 8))
 (segment (start 60 78.5) (end 69 87.5) (width 1) (layer "F.Cu") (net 8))
 (segment (start 87.54 65) (end 87.54 69.96) (width 1) (layer "F.Cu") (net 9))
 (segment (start 77.5 80) (end 77.5 76.17) (width 1) (layer "F.Cu") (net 9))
 (segment (start 77.5 80) (end 77.5 84.175) (width 1) (layer "F.Cu") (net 9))
 (segment (start 87.54 69.96) (end 77.5 80) (width 1) (layer "F.Cu") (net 9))
 (segment (start 87.5 60) (end 82.5 55) (width 1) (layer "B.Cu") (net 9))
 (segment (start 87.5 64.96) (end 87.5 60) (width 1) (layer "B.Cu") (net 9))
 (segment (start 87.54 65) (end 87.5 64.96) (width 1) (layer "B.Cu") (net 9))
 (segment (start 74.72 55) (end 69.96 50.24) (width 1) (layer "B.Cu") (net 9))
 (segment (start 82.5 55) (end 74.72 55) (width 1) (layer "B.Cu") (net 9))
 (segment (start 105 70) (end 101.25 66.25) (width 1) (layer "F.Cu") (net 13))
 (segment (start 101.25 66.25) (end 98.75 66.25) (width 1) (layer "F.Cu") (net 13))
 (segment (start 105 80.85) (end 105 70) (width 1) (layer "F.Cu") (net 13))
 (via (at 98.75 66.25) (size 1.6) (drill 0.8) (layers "F.Cu" "B.Cu") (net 13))
 (segment (start 74.76 52.5) (end 85 52.5) (width 1) (layer "B.Cu") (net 13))
 (segment (start 85 52.5) (end 98.75 66.25) (width 1) (layer "B.Cu") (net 13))
 (segment (start 72.5 50.24) (end 74.76 52.5) (width 1) (layer "B.Cu") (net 13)))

